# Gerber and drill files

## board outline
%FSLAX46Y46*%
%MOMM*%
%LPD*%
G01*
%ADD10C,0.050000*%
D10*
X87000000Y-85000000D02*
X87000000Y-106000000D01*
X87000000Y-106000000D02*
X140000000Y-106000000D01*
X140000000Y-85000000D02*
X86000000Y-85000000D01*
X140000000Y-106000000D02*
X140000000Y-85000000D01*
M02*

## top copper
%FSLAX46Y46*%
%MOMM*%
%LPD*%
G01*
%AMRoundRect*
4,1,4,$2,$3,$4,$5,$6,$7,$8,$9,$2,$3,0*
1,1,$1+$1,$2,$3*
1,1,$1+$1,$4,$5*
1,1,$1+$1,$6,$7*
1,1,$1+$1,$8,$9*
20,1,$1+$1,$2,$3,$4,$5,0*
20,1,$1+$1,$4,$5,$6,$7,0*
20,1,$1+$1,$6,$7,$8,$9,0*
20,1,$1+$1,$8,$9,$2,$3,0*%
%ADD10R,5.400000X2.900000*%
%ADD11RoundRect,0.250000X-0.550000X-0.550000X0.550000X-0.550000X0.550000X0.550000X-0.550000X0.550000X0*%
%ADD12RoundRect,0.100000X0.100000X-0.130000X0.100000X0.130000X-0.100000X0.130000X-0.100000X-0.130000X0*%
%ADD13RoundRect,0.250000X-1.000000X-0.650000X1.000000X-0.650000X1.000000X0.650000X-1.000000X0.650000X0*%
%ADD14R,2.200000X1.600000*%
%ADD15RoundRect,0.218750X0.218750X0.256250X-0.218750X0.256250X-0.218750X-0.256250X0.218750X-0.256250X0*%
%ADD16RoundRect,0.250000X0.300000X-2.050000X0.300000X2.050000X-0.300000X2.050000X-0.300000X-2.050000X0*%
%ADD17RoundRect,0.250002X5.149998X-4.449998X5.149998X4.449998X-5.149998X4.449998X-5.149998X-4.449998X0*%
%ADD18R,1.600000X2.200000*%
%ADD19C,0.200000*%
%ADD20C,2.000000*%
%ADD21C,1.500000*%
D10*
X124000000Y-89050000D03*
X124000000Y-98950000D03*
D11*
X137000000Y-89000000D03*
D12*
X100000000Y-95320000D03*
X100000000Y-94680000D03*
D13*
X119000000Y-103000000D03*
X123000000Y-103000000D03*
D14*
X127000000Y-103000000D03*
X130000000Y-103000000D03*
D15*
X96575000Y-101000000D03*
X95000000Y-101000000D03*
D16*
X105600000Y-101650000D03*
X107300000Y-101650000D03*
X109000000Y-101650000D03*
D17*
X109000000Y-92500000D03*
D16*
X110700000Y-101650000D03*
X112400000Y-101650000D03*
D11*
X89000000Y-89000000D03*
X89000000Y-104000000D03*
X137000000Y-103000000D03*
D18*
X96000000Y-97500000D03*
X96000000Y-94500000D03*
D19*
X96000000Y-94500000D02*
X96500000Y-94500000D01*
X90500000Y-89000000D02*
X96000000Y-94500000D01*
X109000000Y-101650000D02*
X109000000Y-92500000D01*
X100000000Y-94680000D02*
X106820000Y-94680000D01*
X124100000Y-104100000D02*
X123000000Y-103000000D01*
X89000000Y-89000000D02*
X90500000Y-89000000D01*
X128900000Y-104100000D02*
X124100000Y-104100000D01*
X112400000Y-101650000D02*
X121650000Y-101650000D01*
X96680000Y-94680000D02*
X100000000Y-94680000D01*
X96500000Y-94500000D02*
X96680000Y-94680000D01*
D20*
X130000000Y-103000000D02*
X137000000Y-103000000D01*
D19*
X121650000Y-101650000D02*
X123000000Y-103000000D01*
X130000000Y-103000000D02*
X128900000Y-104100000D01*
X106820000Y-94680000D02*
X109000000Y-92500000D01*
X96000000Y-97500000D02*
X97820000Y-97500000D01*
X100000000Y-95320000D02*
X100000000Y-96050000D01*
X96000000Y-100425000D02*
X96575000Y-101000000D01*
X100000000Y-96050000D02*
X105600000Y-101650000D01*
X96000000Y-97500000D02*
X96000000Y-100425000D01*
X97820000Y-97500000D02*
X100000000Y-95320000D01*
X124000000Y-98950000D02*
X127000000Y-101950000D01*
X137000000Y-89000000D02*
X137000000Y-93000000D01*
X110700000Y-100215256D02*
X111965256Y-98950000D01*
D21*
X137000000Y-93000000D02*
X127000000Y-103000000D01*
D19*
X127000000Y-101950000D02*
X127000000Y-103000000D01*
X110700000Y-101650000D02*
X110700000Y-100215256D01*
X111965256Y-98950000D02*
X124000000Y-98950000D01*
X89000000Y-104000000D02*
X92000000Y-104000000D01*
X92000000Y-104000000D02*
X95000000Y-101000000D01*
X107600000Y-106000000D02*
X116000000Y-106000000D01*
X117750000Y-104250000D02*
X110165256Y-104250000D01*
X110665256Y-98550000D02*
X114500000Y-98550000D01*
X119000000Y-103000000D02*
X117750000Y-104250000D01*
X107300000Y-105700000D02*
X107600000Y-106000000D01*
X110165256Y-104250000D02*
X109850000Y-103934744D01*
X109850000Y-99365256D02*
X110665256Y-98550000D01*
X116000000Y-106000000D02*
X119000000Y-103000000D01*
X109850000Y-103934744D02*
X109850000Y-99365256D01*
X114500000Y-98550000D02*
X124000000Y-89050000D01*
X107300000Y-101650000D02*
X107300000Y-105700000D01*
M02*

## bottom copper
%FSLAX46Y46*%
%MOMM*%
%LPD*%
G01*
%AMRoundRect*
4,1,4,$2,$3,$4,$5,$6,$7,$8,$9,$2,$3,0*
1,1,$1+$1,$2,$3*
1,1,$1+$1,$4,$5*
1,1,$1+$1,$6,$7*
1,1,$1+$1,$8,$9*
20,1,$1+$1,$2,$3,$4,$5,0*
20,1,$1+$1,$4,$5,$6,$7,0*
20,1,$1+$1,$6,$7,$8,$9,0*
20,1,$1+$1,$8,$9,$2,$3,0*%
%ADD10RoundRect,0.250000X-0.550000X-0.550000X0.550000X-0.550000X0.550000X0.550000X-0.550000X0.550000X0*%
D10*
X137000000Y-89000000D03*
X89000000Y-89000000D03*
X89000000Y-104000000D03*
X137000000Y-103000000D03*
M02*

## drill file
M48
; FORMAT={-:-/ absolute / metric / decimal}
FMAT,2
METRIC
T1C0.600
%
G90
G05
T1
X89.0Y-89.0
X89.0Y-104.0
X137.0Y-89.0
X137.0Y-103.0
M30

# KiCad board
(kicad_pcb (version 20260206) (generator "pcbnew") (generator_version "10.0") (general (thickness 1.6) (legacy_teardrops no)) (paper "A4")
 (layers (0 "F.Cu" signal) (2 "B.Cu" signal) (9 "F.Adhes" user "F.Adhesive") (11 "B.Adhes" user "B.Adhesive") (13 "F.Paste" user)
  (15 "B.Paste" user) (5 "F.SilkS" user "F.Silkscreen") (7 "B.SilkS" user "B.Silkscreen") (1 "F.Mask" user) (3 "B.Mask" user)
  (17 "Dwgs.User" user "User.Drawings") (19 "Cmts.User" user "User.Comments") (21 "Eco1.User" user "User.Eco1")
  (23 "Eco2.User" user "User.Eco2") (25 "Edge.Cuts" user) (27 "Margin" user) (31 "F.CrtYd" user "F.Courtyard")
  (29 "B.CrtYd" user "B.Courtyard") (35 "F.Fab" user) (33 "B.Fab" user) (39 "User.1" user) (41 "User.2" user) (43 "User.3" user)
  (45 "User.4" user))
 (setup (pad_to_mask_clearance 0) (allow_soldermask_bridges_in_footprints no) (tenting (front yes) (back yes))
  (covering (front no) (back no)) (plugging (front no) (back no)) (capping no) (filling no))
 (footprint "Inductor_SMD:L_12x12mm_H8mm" (layer "F.Cu") (at 124 94 -90)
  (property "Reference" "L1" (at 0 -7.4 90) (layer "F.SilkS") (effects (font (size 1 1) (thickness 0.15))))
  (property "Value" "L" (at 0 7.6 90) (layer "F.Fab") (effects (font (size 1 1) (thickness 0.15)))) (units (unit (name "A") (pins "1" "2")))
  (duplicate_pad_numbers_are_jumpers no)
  (pad "1" smd rect (at -4.95 0 270) (size 2.9 5.4) (layers "F.Cu" "F.Mask" "F.Paste") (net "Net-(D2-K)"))
  (pad "2" smd rect (at 4.95 0 270) (size 2.9 5.4) (layers "F.Cu" "F.Mask" "F.Paste") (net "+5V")))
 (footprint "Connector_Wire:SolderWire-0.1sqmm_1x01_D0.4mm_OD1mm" (layer "F.Cu") (at 137 89)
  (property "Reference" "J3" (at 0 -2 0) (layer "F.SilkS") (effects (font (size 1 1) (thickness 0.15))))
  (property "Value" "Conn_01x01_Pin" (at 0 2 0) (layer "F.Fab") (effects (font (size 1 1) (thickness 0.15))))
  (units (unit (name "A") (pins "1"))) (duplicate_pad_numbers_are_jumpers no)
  (pad "1" thru_hole roundrect (at 0 0) (size 1.6 1.6) (drill 0.6) (layers "*.Cu" "*.Mask") (remove_unused_layers no)
   (roundrect_rratio 0.15625) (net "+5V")))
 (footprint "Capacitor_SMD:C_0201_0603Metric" (layer "F.Cu") (at 100 95 90)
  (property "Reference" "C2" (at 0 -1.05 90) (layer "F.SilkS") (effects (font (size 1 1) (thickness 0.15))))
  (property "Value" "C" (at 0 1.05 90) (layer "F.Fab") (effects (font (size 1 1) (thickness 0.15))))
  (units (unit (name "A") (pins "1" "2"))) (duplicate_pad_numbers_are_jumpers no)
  (pad "" smd roundrect (at -0.345 0 90) (size 0.318 0.36) (layers "F.Paste") (roundrect_rratio 0.25))
  (pad "" smd roundrect (at 0.345 0 90) (size 0.318 0.36) (layers "F.Paste") (roundrect_rratio 0.25))
  (pad "1" smd roundrect (at -0.32 0 90) (size 0.46 0.4) (layers "F.Cu" "F.Mask") (roundrect_rratio 0.25) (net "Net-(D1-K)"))
  (pad "2" smd roundrect (at 0.32 0 90) (size 0.46 0.4) (layers "F.Cu" "F.Mask") (roundrect_rratio 0.25) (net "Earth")))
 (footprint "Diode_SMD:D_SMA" (layer "F.Cu") (at 121 103)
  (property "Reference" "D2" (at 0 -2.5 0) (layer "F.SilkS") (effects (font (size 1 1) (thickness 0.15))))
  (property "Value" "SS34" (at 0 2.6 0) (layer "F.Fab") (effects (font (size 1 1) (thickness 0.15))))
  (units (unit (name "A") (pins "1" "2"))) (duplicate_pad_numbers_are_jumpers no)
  (pad "1" smd roundrect (at -2 0) (size 2.5 1.8) (layers "F.Cu" "F.Mask" "F.Paste") (roundrect_rratio 0.1388888889) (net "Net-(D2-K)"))
  (pad "2" smd roundrect (at 2 0) (size 2.5 1.8) (layers "F.Cu" "F.Mask" "F.Paste") (roundrect_rratio 0.1388888889) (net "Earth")))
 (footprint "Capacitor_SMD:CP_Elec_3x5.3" (layer "F.Cu") (at 128.5 103)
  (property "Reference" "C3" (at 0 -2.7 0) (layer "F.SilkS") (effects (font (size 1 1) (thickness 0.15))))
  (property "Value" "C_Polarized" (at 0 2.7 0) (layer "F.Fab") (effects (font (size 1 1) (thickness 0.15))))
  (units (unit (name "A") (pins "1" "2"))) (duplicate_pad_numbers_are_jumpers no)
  (pad "1" smd rect (at -1.5 0) (size 2.2 1.6) (layers "F.Cu" "F.Mask" "F.Paste") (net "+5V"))
  (pad "2" smd rect (at 1.5 0) (size 2.2 1.6) (layers "F.Cu" "F.Mask" "F.Paste") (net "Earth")))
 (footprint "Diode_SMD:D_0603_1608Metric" (layer "F.Cu") (at 95.7875 101 180)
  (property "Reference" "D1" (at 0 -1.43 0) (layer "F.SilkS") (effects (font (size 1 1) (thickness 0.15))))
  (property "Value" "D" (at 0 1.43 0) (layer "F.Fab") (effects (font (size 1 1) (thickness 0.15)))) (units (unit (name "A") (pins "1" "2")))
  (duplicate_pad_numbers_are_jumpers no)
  (pad "1" smd roundrect (at -0.7875 0 180) (size 0.875 0.95) (layers "F.Cu" "F.Mask" "F.Paste") (roundrect_rratio 0.25) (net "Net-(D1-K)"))
  (pad "2" smd roundrect (at 0.7875 0 180) (size 0.875 0.95) (layers "F.Cu" "F.Mask" "F.Paste") (roundrect_rratio 0.25) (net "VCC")))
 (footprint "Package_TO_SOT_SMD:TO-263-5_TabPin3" (layer "F.Cu") (at 109 94 90)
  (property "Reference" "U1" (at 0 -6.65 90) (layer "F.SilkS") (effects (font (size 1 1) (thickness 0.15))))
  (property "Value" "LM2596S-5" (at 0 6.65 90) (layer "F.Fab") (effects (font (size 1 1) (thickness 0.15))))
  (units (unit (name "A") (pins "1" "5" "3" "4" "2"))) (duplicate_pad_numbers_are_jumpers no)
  (pad "" smd roundrect (at -0.925 -2.775 90) (size 4.55 5.25) (layers "F.Paste") (roundrect_rratio 0.054945))
  (pad "" smd roundrect (at -0.925 2.775 90) (size 4.55 5.25) (layers "F.Paste") (roundrect_rratio 0.054945))
  (pad "" smd roundrect (at 3.925 -2.775 90) (size 4.55 5.25) (layers "F.Paste") (roundrect_rratio 0.054945))
  (pad "" smd roundrect (at 3.925 2.775 90) (size 4.55 5.25) (layers "F.Paste") (roundrect_rratio 0.054945))
  (pad "1" smd roundrect (at -7.65 -3.4 90) (size 4.6 1.1) (layers "F.Cu" "F.Mask" "F.Paste") (roundrect_rratio 0.227273) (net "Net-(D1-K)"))
  (pad "2" smd roundrect (at -7.65 -1.7 90) (size 4.6 1.1) (layers "F.Cu" "F.Mask" "F.Paste") (roundrect_rratio 0.227273) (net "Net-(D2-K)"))
  (pad "3" smd roundrect (at -7.65 0 90) (size 4.6 1.1) (layers "F.Cu" "F.Mask" "F.Paste") (roundrect_rratio 0.227273) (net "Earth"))
  (pad "3" smd roundrect (at 1.5 0 90) (size 9.4 10.8) (layers "F.Cu" "F.Mask") (roundrect_rratio 0.026596) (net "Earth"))
  (pad "4" smd roundrect (at -7.65 1.7 90) (size 4.6 1.1) (layers "F.Cu" "F.Mask" "F.Paste") (roundrect_rratio 0.227273) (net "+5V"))
  (pad "5" smd roundrect (at -7.65 3.4 90) (size 4.6 1.1) (layers "F.Cu" "F.Mask" "F.Paste") (roundrect_rratio 0.227273) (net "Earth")))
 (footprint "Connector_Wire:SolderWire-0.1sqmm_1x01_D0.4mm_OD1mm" (layer "F.Cu") (at 89 89)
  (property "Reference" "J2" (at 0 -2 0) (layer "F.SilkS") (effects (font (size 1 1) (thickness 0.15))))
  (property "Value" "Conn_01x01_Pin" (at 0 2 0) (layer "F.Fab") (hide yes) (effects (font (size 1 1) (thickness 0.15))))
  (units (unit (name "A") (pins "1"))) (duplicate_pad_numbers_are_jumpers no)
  (pad "1" thru_hole roundrect (at 0 0) (size 1.6 1.6) (drill 0.6) (layers "*.Cu" "*.Mask") (remove_unused_layers no)
   (roundrect_rratio 0.15625) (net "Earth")))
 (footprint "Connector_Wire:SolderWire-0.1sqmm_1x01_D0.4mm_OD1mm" (layer "F.Cu") (at 89 104)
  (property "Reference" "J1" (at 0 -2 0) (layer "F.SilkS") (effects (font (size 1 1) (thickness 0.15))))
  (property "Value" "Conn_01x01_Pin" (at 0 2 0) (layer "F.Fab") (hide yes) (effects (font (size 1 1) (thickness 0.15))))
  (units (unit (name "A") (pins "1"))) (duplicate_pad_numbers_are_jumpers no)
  (pad "1" thru_hole roundrect (at 0 0) (size 1.6 1.6) (drill 0.6) (layers "*.Cu" "*.Mask") (remove_unused_layers no)
   (roundrect_rratio 0.15625) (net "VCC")))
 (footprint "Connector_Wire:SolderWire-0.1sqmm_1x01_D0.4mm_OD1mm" (layer "F.Cu") (at 137 103)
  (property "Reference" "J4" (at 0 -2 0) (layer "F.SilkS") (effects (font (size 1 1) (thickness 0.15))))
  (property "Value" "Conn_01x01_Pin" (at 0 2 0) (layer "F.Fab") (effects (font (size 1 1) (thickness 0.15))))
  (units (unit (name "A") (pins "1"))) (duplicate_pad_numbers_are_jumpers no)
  (pad "1" thru_hole roundrect (at 0 0) (size 1.6 1.6) (drill 0.6) (layers "*.Cu" "*.Mask") (remove_unused_layers no)
   (roundrect_rratio 0.15625) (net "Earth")))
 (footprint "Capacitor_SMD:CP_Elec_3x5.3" (layer "F.Cu") (at 96 96 90)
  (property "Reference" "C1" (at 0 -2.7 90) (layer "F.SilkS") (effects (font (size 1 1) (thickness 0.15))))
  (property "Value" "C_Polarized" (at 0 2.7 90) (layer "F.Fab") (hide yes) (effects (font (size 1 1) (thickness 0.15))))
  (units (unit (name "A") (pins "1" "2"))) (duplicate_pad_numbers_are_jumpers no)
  (pad "1" smd rect (at -1.5 0 90) (size 2.2 1.6) (layers "F.Cu" "F.Mask" "F.Paste") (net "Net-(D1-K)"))
  (pad "2" smd rect (at 1.5 0 90) (size 2.2 1.6) (layers "F.Cu" "F.Mask" "F.Paste") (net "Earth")))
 (gr_line (start 87 85) (end 87 106) (stroke (width 0.05) (type default)) (layer "Edge.Cuts"))
 (gr_line (start 87 106) (end 140 106) (stroke (width 0.05) (type default)) (layer "Edge.Cuts"))
 (gr_line (start 140 85) (end 86 85) (stroke (width 0.05) (type default)) (layer "Edge.Cuts"))
 (gr_line (start 140 106) (end 140 85) (stroke (width 0.05) (type default)) (layer "Edge.Cuts"))
 (segment (start 96 94.5) (end 96.5 94.5) (width 0.2) (layer "F.Cu") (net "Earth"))
 (segment (start 90.5 89) (end 96 94.5) (width 0.2) (layer "F.Cu") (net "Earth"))
 (segment (start 109 101.65) (end 109 92.5) (width 0.2) (layer "F.Cu") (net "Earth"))
 (segment (start 100 94.68) (end 106.82 94.68) (width 0.2) (layer "F.Cu") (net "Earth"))
 (segment (start 124.1 104.1) (end 123 103) (width 0.2) (layer "F.Cu") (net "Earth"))
 (segment (start 89 89) (end 90.5 89) (width 0.2) (layer "F.Cu") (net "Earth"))
 (segment (start 128.9 104.1) (end 124.1 104.1) (width 0.2) (layer "F.Cu") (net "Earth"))
 (segment (start 112.4 101.65) (end 121.65 101.65) (width 0.2) (layer "F.Cu") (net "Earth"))
 (segment (start 96.68 94.68) (end 100 94.68) (width 0.2) (layer "F.Cu") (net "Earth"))
 (segment (start 96.5 94.5) (end 96.68 94.68) (width 0.2) (layer "F.Cu") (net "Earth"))
 (segment (start 130 103) (end 137 103) (width 2) (layer "F.Cu") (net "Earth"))
 (segment (start 121.65 101.65) (end 123 103) (width 0.2) (layer "F.Cu") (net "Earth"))
 (segment (start 130 103) (end 128.9 104.1) (width 0.2) (layer "F.Cu") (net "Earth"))
 (segment (start 106.82 94.68) (end 109 92.5) (width 0.2) (layer "F.Cu") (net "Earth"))
 (segment (start 96 97.5) (end 97.82 97.5) (width 0.2) (layer "F.Cu") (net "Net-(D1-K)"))
 (segment (start 100 95.32) (end 100 96.05) (width 0.2) (layer "F.Cu") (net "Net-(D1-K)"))
 (segment (start 96 100.425) (end 96.575 101) (width 0.2) (layer "F.Cu") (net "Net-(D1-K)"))
 (segment (start 100 96.05) (end 105.6 101.65) (width 0.2) (layer "F.Cu") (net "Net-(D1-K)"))
 (segment (start 96 97.5) (end 96 100.425) (width 0.2) (layer "F.Cu") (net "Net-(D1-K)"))
 (segment (start 97.82 97.5) (end 100 95.32) (width 0.2) (layer "F.Cu") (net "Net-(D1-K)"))
 (segment (start 124 98.95) (end 127 101.95) (width 0.2) (layer "F.Cu") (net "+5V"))
 (segment (start 137 89) (end 137 93) (width 0.2) (layer "F.Cu") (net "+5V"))
 (segment (start 110.7 100.215256) (end 111.965256 98.95) (width 0.2) (layer "F.Cu") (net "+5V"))
 (segment (start 137 93) (end 127 103) (width 1.5) (layer "F.Cu") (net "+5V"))
 (segment (start 127 101.95) (end 127 103) (width 0.2) (layer "F.Cu") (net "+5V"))
 (segment (start 110.7 101.65) (end 110.7 100.215256) (width 0.2) (layer "F.Cu") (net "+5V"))
 (segment (start 111.965256 98.95) (end 124 98.95) (width 0.2) (layer "F.Cu") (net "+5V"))
 (segment (start 89 104) (end 92 104) (width 0.2) (layer "F.Cu") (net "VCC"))
 (segment (start 92 104) (end 95 101) (width 0.2) (layer "F.Cu") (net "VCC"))
 (segment (start 107.6 106) (end 116 106) (width 0.2) (layer "F.Cu") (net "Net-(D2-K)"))
 (segment (start 117.75 104.25) (end 110.165256 104.25) (width 0.2) (layer "F.Cu") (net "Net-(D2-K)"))
 (segment (start 110.665256 98.55) (end 114.5 98.55) (width 0.2) (layer "F.Cu") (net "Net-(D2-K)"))
 (segment (start 119 103) (end 117.75 104.25) (width 0.2) (layer "F.Cu") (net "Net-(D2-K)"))
 (segment (start 107.3 105.7) (end 107.6 106) (width 0.2) (layer "F.Cu") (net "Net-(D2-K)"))
 (segment (start 110.165256 104.25) (end 109.85 103.934744) (width 0.2) (layer "F.Cu") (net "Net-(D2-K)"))
 (segment (start 109.85 99.365256) (end 110.665256 98.55) (width 0.2) (layer "F.Cu") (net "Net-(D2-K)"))
 (segment (start 116 106) (end 119 103) (width 0.2) (layer "F.Cu") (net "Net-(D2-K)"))
 (segment (start 109.85 103.934744) (end 109.85 99.365256) (width 0.2) (layer "F.Cu") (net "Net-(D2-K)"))
 (segment (start 114.5 98.55) (end 124 89.05) (width 0.2) (layer "F.Cu") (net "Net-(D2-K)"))
 (segment (start 107.3 101.65) (end 107.3 105.7) (width 0.2) (layer "F.Cu") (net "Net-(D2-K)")))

